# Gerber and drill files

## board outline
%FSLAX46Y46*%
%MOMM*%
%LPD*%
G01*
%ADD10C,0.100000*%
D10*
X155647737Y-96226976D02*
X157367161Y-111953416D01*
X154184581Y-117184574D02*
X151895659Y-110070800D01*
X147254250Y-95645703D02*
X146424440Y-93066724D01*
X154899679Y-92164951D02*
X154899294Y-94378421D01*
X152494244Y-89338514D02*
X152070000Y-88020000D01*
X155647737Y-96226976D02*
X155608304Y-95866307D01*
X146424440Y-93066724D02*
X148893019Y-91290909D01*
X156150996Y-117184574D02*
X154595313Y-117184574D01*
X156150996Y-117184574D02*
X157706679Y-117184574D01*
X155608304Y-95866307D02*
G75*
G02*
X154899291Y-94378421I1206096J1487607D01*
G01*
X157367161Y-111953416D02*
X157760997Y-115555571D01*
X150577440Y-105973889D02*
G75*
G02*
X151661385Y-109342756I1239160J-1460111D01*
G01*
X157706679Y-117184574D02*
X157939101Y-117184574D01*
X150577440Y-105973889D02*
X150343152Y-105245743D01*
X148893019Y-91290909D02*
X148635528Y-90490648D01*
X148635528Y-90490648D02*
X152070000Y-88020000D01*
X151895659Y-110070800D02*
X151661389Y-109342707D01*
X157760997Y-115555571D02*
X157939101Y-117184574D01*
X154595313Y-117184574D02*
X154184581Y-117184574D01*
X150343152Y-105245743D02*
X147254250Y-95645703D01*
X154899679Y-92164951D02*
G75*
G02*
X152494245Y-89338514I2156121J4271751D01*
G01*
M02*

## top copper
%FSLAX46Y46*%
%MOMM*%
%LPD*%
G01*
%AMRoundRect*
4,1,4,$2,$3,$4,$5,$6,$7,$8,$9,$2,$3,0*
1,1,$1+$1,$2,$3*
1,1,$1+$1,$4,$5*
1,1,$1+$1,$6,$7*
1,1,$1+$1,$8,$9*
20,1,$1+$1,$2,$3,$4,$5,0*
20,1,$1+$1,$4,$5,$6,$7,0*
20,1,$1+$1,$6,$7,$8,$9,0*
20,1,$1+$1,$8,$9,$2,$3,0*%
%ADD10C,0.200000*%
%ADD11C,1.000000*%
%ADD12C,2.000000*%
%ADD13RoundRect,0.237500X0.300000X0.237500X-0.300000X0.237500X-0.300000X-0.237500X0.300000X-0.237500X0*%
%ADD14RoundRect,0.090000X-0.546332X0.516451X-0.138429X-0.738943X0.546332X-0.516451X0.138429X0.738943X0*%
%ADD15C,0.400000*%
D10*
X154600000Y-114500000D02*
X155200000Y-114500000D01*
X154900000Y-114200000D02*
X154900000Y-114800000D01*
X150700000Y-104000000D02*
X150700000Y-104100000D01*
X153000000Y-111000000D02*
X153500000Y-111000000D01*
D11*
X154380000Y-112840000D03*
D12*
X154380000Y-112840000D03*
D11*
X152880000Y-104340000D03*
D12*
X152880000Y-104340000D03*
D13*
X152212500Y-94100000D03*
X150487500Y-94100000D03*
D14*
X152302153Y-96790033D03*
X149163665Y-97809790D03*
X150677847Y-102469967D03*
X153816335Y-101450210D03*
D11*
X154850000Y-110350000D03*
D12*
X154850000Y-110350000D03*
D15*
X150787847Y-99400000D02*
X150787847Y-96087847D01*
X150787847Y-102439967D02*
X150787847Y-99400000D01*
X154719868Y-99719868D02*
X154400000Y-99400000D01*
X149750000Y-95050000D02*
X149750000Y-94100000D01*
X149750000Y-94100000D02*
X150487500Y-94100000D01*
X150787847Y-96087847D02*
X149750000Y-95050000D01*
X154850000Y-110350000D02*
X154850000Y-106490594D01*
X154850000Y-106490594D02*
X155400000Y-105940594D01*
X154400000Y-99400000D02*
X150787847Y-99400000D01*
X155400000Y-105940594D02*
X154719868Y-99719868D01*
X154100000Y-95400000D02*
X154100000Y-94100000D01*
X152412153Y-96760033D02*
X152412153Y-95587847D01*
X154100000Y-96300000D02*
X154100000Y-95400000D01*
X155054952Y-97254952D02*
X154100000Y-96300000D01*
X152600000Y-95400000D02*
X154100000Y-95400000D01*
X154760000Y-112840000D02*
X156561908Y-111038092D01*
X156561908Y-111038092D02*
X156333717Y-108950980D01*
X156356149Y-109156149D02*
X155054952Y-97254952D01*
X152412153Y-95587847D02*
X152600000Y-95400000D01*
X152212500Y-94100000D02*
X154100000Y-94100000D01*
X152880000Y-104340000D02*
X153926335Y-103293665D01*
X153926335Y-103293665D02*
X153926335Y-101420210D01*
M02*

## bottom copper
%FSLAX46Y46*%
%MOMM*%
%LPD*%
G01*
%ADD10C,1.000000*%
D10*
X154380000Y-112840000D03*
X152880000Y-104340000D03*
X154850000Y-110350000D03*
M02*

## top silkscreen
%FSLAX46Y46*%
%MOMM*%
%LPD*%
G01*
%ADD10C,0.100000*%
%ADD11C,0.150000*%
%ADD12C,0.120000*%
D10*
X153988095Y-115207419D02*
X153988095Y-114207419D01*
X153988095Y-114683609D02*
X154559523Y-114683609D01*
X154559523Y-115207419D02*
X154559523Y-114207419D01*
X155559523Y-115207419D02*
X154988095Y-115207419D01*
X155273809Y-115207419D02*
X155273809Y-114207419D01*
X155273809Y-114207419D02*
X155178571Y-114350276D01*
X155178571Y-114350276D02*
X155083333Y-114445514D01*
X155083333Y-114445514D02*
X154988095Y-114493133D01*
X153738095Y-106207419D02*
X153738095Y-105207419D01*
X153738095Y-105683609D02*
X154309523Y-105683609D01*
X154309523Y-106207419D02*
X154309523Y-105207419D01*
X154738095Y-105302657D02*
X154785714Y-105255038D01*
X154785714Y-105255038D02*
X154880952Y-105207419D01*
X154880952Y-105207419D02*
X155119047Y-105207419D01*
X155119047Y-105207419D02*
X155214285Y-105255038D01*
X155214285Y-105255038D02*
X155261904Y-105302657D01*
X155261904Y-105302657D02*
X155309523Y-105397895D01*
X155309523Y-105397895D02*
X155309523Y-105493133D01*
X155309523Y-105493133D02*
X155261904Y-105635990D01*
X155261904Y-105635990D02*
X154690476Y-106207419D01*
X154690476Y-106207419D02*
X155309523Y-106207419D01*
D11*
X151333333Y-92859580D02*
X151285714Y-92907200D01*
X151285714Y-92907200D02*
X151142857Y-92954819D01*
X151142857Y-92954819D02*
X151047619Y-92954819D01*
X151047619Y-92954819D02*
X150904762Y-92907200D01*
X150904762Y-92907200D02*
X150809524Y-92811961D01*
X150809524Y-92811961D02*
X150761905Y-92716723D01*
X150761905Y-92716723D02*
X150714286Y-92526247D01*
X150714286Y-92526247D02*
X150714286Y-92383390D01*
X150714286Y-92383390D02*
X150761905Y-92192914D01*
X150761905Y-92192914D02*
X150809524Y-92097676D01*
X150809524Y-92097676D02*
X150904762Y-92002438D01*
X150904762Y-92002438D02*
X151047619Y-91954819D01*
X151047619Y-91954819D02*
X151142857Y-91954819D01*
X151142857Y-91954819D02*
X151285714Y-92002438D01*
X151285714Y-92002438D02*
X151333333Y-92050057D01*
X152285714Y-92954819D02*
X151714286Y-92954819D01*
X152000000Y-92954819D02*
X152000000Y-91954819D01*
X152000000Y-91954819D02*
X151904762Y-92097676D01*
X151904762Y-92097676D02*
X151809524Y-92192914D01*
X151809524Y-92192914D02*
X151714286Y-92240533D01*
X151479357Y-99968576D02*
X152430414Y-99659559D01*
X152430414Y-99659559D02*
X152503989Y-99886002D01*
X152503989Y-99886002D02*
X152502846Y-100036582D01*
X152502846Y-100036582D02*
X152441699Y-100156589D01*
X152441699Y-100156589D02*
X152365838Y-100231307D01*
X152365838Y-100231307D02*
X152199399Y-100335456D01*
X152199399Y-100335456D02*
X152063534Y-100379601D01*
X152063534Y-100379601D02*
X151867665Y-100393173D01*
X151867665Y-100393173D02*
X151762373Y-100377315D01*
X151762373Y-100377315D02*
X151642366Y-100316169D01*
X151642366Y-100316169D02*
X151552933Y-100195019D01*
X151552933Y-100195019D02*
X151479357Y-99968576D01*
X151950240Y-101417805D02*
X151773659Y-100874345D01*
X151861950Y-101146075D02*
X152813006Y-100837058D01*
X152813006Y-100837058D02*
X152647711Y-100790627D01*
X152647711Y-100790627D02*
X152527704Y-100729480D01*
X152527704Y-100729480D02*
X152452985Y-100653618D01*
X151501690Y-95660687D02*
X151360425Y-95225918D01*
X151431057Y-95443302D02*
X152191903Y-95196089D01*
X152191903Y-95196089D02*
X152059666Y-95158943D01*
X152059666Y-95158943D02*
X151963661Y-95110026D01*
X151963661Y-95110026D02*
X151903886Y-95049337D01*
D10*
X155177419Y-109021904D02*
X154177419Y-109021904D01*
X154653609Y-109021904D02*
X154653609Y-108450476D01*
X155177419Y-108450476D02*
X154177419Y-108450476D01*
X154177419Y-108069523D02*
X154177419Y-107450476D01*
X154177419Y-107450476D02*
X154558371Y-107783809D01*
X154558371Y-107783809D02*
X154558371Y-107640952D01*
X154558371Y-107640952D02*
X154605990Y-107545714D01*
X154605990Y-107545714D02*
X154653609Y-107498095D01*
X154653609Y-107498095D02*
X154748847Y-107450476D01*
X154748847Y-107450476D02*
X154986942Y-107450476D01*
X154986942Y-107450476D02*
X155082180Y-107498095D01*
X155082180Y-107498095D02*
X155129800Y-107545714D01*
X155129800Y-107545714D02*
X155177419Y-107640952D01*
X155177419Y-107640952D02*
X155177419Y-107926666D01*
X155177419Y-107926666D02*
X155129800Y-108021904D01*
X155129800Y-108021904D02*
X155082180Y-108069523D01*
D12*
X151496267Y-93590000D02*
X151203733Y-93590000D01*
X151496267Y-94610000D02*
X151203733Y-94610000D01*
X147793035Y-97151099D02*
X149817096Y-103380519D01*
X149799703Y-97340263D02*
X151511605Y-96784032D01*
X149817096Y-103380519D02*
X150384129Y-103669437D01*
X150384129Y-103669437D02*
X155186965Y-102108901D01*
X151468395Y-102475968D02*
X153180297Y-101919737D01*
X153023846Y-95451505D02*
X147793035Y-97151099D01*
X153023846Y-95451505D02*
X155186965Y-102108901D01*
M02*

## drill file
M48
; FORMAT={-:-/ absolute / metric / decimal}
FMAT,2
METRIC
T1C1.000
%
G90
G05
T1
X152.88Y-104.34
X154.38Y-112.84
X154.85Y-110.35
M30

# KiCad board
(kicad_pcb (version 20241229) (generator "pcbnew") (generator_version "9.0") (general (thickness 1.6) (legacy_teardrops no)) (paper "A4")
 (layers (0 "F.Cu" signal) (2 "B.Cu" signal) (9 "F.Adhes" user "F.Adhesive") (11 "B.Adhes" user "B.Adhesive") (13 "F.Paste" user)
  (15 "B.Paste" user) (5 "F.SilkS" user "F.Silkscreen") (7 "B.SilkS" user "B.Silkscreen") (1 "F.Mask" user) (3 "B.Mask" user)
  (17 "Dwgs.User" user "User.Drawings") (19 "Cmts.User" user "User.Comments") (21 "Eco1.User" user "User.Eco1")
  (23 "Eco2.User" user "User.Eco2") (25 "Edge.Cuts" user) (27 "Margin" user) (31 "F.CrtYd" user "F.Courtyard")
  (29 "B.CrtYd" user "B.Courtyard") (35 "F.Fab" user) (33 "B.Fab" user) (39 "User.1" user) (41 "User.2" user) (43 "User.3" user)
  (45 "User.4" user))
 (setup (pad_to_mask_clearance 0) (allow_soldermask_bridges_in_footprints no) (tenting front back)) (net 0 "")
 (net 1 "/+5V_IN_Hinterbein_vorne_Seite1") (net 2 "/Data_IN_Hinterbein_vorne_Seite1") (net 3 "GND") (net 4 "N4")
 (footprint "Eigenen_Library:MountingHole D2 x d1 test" (layer "F.Cu") (at 154.38 112.84)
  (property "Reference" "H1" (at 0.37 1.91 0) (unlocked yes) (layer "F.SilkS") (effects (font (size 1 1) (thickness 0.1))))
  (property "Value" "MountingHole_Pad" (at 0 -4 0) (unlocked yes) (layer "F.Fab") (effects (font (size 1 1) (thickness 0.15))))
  (pad "1" thru_hole circle (at 0 0) (size 1 1) (drill 1) (layers "*.Cu" "*.Mask") (remove_unused_layers no)
   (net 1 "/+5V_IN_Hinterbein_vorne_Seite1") (zone_connect 2))
  (pad "1" connect circle (at 0 0) (size 2 2) (layers "F.Cu" "F.Mask") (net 1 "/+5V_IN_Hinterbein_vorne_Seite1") (zone_connect 2)))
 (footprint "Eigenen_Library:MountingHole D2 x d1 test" (layer "F.Cu") (at 152.88 104.34)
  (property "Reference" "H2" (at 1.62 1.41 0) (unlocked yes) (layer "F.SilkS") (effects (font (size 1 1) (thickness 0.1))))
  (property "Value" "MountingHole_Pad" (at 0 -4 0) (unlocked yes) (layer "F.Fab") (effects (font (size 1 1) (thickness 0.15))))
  (pad "1" thru_hole circle (at 0 0) (size 1 1) (drill 1) (layers "*.Cu" "*.Mask") (remove_unused_layers no)
   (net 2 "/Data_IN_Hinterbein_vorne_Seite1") (zone_connect 2))
  (pad "1" connect circle (at 0 0) (size 2 2) (layers "F.Cu" "F.Mask") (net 2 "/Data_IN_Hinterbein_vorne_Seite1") (zone_connect 2)))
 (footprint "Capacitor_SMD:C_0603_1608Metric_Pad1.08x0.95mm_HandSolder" (layer "F.Cu") (at 151.35 94.1 180)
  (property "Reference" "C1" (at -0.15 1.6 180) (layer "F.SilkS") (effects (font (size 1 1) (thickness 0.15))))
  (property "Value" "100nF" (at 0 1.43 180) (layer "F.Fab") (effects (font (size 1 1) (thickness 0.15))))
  (fp_line (start -0.146267 0.51) (end 0.146267 0.51) (stroke (width 0.12) (type solid)) (layer "F.SilkS"))
  (fp_line (start -0.146267 -0.51) (end 0.146267 -0.51) (stroke (width 0.12) (type solid)) (layer "F.SilkS"))
  (pad "1" smd roundrect (at -0.8625 0 180) (size 1.075 0.95) (layers "F.Cu" "F.Mask" "F.Paste") (roundrect_rratio 0.25)
   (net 1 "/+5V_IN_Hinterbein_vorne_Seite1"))
  (pad "2" smd roundrect (at 0.8625 0 180) (size 1.075 0.95) (layers "F.Cu" "F.Mask" "F.Paste") (roundrect_rratio 0.25) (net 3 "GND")))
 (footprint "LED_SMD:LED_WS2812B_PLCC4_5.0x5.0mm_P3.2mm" (layer "F.Cu") (at 151.49 99.63 -72)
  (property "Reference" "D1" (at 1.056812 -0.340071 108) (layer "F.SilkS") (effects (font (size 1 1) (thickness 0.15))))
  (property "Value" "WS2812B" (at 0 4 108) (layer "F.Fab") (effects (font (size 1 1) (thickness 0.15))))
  (fp_line (start -3.5 2.75) (end 3.05 2.75) (stroke (width 0.12) (type solid)) (layer "F.SilkS"))
  (fp_line (start -2.7 0.9) (end -2.7 -0.9) (stroke (width 0.12) (type default)) (layer "F.SilkS"))
  (fp_line (start 3.05 2.75) (end 3.5 2.300001) (stroke (width 0.12) (type default)) (layer "F.SilkS"))
  (fp_line (start 3.5 2.300001) (end 3.5 -2.75) (stroke (width 0.12) (type default)) (layer "F.SilkS"))
  (fp_line (start 2.7 0.9) (end 2.7 -0.9) (stroke (width 0.12) (type default)) (layer "F.SilkS"))
  (fp_line (start -3.5 -2.75) (end -3.5 2.75) (stroke (width 0.12) (type default)) (layer "F.SilkS"))
  (fp_line (start -3.5 -2.75) (end 3.5 -2.75) (stroke (width 0.12) (type solid)) (layer "F.SilkS"))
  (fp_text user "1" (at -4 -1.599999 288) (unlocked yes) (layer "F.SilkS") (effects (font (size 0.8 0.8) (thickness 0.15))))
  (pad "1" smd roundrect (at -2.45 -1.650001 288) (size 1.5 0.9) (layers "F.Cu" "F.Mask" "F.Paste") (roundrect_rratio 0.1)
   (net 1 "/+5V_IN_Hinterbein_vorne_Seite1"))
  (pad "2" smd roundrect (at -2.45 1.65 288) (size 1.5 0.9) (layers "F.Cu" "F.Mask" "F.Paste") (roundrect_rratio 0.1) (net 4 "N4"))
  (pad "3" smd roundrect (at 2.45 1.650001 288) (size 1.5 0.9) (layers "F.Cu" "F.Mask" "F.Paste") (roundrect_rratio 0.1) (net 3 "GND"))
  (pad "4" smd roundrect (at 2.45 -1.65 288) (size 1.5 0.9) (layers "F.Cu" "F.Mask" "F.Paste") (roundrect_rratio 0.1)
   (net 2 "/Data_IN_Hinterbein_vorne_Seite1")))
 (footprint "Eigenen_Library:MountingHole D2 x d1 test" (layer "F.Cu") (at 154.85 110.35)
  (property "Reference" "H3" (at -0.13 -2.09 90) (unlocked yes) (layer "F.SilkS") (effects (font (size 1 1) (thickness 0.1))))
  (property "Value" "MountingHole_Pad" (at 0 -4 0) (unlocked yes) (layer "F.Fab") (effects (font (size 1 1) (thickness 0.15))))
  (pad "1" thru_hole circle (at 0 0) (size 1 1) (drill 1) (layers "*.Cu" "*.Mask") (remove_unused_layers no) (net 3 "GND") (zone_connect 2))
  (pad "1" connect circle (at 0 0) (size 2 2) (layers "F.Cu" "F.Mask") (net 3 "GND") (zone_connect 2)))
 (gr_line (start 154.6 114.5) (end 155.2 114.5) (stroke (width 0.2) (type default)) (layer "F.Cu"))
 (gr_line (start 154.9 114.2) (end 154.9 114.8) (stroke (width 0.2) (type default)) (layer "F.Cu"))
 (gr_line (start 150.7 104) (end 150.7 104.1) (stroke (width 0.2) (type default)) (layer "F.Cu"))
 (gr_line (start 153 111) (end 153.5 111) (stroke (width 0.2) (type default)) (layer "F.Cu"))
 (gr_line (start 155.647737 96.226976) (end 157.367161 111.953416) (stroke (width 0.1) (type default)) (locked yes) (layer "Edge.Cuts"))
 (gr_line (start 154.184581 117.184574) (end 151.895659 110.0708) (stroke (width 0.1) (type default)) (locked yes) (layer "Edge.Cuts"))
 (gr_line (start 147.25425 95.645703) (end 146.42444 93.066724) (stroke (width 0.1) (type default)) (locked yes) (layer "Edge.Cuts"))
 (gr_line (start 154.899679 92.164951) (end 154.899294 94.378421) (stroke (width 0.1) (type default)) (locked yes) (layer "Edge.Cuts"))
 (gr_line (start 152.494244 89.338514) (end 152.07 88.02) (stroke (width 0.1) (type default)) (locked yes) (layer "Edge.Cuts"))
 (gr_line (start 155.647737 96.226976) (end 155.608304 95.866307) (stroke (width 0.1) (type default)) (locked yes) (layer "Edge.Cuts"))
 (gr_line (start 146.42444 93.066724) (end 148.893019 91.290909) (stroke (width 0.1) (type default)) (locked yes) (layer "Edge.Cuts"))
 (gr_line (start 156.150996 117.184574) (end 154.595313 117.184574) (stroke (width 0.1) (type default)) (locked yes) (layer "Edge.Cuts"))
 (gr_line (start 156.150996 117.184574) (end 157.706679 117.184574) (stroke (width 0.1) (type default)) (locked yes) (layer "Edge.Cuts"))
 (gr_arc (start 155.608304 95.866307) (mid 155.085545 95.202543) (end 154.899294 94.378421) (stroke (width 0.1) (type default)) (locked yes)
  (layer "Edge.Cuts"))
 (gr_line (start 157.367161 111.953416) (end 157.760997 115.555571) (stroke (width 0.1) (type default)) (locked yes) (layer "Edge.Cuts"))
 (gr_arc (start 150.57744 105.973889) (mid 153.639581 106.847423) (end 151.661389 109.342707) (stroke (width 0.1) (type default))
  (locked yes) (layer "Edge.Cuts"))
 (gr_line (start 157.706679 117.184574) (end 157.939101 117.184574) (stroke (width 0.1) (type default)) (locked yes) (layer "Edge.Cuts"))
 (gr_line (start 150.57744 105.973889) (end 150.343152 105.245743) (stroke (width 0.1) (type default)) (locked yes) (layer "Edge.Cuts"))
 (gr_line (start 148.893019 91.290909) (end 148.635528 90.490648) (stroke (width 0.1) (type default)) (locked yes) (layer "Edge.Cuts"))
 (gr_line (start 148.635528 90.490648) (end 152.07 88.02) (stroke (width 0.1) (type default)) (locked yes) (layer "Edge.Cuts"))
 (gr_line (start 151.895659 110.0708) (end 151.661389 109.342707) (stroke (width 0.1) (type default)) (locked yes) (layer "Edge.Cuts"))
 (gr_line (start 157.760997 115.555571) (end 157.939101 117.184574) (stroke (width 0.1) (type default)) (locked yes) (layer "Edge.Cuts"))
 (gr_line (start 154.595313 117.184574) (end 154.184581 117.184574) (stroke (width 0.1) (type default)) (locked yes) (layer "Edge.Cuts"))
 (gr_line (start 150.343152 105.245743) (end 147.25425 95.645703) (stroke (width 0.1) (type default)) (locked yes) (layer "Edge.Cuts"))
 (gr_arc (start 154.899679 92.164951) (mid 153.418749 91.002631) (end 152.494244 89.338514) (stroke (width 0.1) (type default)) (locked yes)
  (layer "Edge.Cuts"))
 (segment (start 150.787847 99.4) (end 150.787847 96.087847) (width 0.4) (layer "F.Cu") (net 3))
 (segment (start 150.787847 102.439967) (end 150.787847 99.4) (width 0.4) (layer "F.Cu") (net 3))
 (segment (start 154.719868 99.719868) (end 154.4 99.4) (width 0.4) (layer "F.Cu") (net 3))
 (segment (start 149.75 95.05) (end 149.75 94.1) (width 0.4) (layer "F.Cu") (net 3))
 (segment (start 149.75 94.1) (end 150.4875 94.1) (width 0.4) (layer "F.Cu") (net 3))
 (segment (start 150.787847 96.087847) (end 149.75 95.05) (width 0.4) (layer "F.Cu") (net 3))
 (segment (start 154.85 110.35) (end 154.85 106.490594) (width 0.4) (layer "F.Cu") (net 3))
 (segment (start 154.85 106.490594) (end 155.4 105.940594) (width 0.4) (layer "F.Cu") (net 3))
 (segment (start 154.4 99.4) (end 150.787847 99.4) (width 0.4) (layer "F.Cu") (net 3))
 (segment (start 155.4 105.940594) (end 154.719868 99.719868) (width 0.4) (layer "F.Cu") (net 3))
 (segment (start 154.1 95.4) (end 154.1 94.1) (width 0.4) (layer "F.Cu") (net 1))
 (segment (start 152.412153 96.760033) (end 152.412153 95.587847) (width 0.4) (layer "F.Cu") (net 1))
 (segment (start 154.1 96.3) (end 154.1 95.4) (width 0.4) (layer "F.Cu") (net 1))
 (segment (start 155.054952 97.254952) (end 154.1 96.3) (width 0.4) (layer "F.Cu") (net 1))
 (segment (start 152.6 95.4) (end 154.1 95.4) (width 0.4) (layer "F.Cu") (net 1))
 (segment (start 154.76 112.84) (end 156.561908 111.038092) (width 0.4) (layer "F.Cu") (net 1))
 (segment (start 156.561908 111.038092) (end 156.333717 108.95098) (width 0.4) (layer "F.Cu") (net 1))
 (segment (start 156.356149 109.156149) (end 155.054952 97.254952) (width 0.4) (layer "F.Cu") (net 1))
 (segment (start 152.412153 95.587847) (end 152.6 95.4) (width 0.4) (layer "F.Cu") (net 1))
 (segment (start 152.2125 94.1) (end 154.1 94.1) (width 0.4) (layer "F.Cu") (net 1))
 (segment (start 152.88 104.34) (end 153.926335 103.293665) (width 0.4) (layer "F.Cu") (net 2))
 (segment (start 153.926335 103.293665) (end 153.926335 101.42021) (width 0.4) (layer "F.Cu") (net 2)))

